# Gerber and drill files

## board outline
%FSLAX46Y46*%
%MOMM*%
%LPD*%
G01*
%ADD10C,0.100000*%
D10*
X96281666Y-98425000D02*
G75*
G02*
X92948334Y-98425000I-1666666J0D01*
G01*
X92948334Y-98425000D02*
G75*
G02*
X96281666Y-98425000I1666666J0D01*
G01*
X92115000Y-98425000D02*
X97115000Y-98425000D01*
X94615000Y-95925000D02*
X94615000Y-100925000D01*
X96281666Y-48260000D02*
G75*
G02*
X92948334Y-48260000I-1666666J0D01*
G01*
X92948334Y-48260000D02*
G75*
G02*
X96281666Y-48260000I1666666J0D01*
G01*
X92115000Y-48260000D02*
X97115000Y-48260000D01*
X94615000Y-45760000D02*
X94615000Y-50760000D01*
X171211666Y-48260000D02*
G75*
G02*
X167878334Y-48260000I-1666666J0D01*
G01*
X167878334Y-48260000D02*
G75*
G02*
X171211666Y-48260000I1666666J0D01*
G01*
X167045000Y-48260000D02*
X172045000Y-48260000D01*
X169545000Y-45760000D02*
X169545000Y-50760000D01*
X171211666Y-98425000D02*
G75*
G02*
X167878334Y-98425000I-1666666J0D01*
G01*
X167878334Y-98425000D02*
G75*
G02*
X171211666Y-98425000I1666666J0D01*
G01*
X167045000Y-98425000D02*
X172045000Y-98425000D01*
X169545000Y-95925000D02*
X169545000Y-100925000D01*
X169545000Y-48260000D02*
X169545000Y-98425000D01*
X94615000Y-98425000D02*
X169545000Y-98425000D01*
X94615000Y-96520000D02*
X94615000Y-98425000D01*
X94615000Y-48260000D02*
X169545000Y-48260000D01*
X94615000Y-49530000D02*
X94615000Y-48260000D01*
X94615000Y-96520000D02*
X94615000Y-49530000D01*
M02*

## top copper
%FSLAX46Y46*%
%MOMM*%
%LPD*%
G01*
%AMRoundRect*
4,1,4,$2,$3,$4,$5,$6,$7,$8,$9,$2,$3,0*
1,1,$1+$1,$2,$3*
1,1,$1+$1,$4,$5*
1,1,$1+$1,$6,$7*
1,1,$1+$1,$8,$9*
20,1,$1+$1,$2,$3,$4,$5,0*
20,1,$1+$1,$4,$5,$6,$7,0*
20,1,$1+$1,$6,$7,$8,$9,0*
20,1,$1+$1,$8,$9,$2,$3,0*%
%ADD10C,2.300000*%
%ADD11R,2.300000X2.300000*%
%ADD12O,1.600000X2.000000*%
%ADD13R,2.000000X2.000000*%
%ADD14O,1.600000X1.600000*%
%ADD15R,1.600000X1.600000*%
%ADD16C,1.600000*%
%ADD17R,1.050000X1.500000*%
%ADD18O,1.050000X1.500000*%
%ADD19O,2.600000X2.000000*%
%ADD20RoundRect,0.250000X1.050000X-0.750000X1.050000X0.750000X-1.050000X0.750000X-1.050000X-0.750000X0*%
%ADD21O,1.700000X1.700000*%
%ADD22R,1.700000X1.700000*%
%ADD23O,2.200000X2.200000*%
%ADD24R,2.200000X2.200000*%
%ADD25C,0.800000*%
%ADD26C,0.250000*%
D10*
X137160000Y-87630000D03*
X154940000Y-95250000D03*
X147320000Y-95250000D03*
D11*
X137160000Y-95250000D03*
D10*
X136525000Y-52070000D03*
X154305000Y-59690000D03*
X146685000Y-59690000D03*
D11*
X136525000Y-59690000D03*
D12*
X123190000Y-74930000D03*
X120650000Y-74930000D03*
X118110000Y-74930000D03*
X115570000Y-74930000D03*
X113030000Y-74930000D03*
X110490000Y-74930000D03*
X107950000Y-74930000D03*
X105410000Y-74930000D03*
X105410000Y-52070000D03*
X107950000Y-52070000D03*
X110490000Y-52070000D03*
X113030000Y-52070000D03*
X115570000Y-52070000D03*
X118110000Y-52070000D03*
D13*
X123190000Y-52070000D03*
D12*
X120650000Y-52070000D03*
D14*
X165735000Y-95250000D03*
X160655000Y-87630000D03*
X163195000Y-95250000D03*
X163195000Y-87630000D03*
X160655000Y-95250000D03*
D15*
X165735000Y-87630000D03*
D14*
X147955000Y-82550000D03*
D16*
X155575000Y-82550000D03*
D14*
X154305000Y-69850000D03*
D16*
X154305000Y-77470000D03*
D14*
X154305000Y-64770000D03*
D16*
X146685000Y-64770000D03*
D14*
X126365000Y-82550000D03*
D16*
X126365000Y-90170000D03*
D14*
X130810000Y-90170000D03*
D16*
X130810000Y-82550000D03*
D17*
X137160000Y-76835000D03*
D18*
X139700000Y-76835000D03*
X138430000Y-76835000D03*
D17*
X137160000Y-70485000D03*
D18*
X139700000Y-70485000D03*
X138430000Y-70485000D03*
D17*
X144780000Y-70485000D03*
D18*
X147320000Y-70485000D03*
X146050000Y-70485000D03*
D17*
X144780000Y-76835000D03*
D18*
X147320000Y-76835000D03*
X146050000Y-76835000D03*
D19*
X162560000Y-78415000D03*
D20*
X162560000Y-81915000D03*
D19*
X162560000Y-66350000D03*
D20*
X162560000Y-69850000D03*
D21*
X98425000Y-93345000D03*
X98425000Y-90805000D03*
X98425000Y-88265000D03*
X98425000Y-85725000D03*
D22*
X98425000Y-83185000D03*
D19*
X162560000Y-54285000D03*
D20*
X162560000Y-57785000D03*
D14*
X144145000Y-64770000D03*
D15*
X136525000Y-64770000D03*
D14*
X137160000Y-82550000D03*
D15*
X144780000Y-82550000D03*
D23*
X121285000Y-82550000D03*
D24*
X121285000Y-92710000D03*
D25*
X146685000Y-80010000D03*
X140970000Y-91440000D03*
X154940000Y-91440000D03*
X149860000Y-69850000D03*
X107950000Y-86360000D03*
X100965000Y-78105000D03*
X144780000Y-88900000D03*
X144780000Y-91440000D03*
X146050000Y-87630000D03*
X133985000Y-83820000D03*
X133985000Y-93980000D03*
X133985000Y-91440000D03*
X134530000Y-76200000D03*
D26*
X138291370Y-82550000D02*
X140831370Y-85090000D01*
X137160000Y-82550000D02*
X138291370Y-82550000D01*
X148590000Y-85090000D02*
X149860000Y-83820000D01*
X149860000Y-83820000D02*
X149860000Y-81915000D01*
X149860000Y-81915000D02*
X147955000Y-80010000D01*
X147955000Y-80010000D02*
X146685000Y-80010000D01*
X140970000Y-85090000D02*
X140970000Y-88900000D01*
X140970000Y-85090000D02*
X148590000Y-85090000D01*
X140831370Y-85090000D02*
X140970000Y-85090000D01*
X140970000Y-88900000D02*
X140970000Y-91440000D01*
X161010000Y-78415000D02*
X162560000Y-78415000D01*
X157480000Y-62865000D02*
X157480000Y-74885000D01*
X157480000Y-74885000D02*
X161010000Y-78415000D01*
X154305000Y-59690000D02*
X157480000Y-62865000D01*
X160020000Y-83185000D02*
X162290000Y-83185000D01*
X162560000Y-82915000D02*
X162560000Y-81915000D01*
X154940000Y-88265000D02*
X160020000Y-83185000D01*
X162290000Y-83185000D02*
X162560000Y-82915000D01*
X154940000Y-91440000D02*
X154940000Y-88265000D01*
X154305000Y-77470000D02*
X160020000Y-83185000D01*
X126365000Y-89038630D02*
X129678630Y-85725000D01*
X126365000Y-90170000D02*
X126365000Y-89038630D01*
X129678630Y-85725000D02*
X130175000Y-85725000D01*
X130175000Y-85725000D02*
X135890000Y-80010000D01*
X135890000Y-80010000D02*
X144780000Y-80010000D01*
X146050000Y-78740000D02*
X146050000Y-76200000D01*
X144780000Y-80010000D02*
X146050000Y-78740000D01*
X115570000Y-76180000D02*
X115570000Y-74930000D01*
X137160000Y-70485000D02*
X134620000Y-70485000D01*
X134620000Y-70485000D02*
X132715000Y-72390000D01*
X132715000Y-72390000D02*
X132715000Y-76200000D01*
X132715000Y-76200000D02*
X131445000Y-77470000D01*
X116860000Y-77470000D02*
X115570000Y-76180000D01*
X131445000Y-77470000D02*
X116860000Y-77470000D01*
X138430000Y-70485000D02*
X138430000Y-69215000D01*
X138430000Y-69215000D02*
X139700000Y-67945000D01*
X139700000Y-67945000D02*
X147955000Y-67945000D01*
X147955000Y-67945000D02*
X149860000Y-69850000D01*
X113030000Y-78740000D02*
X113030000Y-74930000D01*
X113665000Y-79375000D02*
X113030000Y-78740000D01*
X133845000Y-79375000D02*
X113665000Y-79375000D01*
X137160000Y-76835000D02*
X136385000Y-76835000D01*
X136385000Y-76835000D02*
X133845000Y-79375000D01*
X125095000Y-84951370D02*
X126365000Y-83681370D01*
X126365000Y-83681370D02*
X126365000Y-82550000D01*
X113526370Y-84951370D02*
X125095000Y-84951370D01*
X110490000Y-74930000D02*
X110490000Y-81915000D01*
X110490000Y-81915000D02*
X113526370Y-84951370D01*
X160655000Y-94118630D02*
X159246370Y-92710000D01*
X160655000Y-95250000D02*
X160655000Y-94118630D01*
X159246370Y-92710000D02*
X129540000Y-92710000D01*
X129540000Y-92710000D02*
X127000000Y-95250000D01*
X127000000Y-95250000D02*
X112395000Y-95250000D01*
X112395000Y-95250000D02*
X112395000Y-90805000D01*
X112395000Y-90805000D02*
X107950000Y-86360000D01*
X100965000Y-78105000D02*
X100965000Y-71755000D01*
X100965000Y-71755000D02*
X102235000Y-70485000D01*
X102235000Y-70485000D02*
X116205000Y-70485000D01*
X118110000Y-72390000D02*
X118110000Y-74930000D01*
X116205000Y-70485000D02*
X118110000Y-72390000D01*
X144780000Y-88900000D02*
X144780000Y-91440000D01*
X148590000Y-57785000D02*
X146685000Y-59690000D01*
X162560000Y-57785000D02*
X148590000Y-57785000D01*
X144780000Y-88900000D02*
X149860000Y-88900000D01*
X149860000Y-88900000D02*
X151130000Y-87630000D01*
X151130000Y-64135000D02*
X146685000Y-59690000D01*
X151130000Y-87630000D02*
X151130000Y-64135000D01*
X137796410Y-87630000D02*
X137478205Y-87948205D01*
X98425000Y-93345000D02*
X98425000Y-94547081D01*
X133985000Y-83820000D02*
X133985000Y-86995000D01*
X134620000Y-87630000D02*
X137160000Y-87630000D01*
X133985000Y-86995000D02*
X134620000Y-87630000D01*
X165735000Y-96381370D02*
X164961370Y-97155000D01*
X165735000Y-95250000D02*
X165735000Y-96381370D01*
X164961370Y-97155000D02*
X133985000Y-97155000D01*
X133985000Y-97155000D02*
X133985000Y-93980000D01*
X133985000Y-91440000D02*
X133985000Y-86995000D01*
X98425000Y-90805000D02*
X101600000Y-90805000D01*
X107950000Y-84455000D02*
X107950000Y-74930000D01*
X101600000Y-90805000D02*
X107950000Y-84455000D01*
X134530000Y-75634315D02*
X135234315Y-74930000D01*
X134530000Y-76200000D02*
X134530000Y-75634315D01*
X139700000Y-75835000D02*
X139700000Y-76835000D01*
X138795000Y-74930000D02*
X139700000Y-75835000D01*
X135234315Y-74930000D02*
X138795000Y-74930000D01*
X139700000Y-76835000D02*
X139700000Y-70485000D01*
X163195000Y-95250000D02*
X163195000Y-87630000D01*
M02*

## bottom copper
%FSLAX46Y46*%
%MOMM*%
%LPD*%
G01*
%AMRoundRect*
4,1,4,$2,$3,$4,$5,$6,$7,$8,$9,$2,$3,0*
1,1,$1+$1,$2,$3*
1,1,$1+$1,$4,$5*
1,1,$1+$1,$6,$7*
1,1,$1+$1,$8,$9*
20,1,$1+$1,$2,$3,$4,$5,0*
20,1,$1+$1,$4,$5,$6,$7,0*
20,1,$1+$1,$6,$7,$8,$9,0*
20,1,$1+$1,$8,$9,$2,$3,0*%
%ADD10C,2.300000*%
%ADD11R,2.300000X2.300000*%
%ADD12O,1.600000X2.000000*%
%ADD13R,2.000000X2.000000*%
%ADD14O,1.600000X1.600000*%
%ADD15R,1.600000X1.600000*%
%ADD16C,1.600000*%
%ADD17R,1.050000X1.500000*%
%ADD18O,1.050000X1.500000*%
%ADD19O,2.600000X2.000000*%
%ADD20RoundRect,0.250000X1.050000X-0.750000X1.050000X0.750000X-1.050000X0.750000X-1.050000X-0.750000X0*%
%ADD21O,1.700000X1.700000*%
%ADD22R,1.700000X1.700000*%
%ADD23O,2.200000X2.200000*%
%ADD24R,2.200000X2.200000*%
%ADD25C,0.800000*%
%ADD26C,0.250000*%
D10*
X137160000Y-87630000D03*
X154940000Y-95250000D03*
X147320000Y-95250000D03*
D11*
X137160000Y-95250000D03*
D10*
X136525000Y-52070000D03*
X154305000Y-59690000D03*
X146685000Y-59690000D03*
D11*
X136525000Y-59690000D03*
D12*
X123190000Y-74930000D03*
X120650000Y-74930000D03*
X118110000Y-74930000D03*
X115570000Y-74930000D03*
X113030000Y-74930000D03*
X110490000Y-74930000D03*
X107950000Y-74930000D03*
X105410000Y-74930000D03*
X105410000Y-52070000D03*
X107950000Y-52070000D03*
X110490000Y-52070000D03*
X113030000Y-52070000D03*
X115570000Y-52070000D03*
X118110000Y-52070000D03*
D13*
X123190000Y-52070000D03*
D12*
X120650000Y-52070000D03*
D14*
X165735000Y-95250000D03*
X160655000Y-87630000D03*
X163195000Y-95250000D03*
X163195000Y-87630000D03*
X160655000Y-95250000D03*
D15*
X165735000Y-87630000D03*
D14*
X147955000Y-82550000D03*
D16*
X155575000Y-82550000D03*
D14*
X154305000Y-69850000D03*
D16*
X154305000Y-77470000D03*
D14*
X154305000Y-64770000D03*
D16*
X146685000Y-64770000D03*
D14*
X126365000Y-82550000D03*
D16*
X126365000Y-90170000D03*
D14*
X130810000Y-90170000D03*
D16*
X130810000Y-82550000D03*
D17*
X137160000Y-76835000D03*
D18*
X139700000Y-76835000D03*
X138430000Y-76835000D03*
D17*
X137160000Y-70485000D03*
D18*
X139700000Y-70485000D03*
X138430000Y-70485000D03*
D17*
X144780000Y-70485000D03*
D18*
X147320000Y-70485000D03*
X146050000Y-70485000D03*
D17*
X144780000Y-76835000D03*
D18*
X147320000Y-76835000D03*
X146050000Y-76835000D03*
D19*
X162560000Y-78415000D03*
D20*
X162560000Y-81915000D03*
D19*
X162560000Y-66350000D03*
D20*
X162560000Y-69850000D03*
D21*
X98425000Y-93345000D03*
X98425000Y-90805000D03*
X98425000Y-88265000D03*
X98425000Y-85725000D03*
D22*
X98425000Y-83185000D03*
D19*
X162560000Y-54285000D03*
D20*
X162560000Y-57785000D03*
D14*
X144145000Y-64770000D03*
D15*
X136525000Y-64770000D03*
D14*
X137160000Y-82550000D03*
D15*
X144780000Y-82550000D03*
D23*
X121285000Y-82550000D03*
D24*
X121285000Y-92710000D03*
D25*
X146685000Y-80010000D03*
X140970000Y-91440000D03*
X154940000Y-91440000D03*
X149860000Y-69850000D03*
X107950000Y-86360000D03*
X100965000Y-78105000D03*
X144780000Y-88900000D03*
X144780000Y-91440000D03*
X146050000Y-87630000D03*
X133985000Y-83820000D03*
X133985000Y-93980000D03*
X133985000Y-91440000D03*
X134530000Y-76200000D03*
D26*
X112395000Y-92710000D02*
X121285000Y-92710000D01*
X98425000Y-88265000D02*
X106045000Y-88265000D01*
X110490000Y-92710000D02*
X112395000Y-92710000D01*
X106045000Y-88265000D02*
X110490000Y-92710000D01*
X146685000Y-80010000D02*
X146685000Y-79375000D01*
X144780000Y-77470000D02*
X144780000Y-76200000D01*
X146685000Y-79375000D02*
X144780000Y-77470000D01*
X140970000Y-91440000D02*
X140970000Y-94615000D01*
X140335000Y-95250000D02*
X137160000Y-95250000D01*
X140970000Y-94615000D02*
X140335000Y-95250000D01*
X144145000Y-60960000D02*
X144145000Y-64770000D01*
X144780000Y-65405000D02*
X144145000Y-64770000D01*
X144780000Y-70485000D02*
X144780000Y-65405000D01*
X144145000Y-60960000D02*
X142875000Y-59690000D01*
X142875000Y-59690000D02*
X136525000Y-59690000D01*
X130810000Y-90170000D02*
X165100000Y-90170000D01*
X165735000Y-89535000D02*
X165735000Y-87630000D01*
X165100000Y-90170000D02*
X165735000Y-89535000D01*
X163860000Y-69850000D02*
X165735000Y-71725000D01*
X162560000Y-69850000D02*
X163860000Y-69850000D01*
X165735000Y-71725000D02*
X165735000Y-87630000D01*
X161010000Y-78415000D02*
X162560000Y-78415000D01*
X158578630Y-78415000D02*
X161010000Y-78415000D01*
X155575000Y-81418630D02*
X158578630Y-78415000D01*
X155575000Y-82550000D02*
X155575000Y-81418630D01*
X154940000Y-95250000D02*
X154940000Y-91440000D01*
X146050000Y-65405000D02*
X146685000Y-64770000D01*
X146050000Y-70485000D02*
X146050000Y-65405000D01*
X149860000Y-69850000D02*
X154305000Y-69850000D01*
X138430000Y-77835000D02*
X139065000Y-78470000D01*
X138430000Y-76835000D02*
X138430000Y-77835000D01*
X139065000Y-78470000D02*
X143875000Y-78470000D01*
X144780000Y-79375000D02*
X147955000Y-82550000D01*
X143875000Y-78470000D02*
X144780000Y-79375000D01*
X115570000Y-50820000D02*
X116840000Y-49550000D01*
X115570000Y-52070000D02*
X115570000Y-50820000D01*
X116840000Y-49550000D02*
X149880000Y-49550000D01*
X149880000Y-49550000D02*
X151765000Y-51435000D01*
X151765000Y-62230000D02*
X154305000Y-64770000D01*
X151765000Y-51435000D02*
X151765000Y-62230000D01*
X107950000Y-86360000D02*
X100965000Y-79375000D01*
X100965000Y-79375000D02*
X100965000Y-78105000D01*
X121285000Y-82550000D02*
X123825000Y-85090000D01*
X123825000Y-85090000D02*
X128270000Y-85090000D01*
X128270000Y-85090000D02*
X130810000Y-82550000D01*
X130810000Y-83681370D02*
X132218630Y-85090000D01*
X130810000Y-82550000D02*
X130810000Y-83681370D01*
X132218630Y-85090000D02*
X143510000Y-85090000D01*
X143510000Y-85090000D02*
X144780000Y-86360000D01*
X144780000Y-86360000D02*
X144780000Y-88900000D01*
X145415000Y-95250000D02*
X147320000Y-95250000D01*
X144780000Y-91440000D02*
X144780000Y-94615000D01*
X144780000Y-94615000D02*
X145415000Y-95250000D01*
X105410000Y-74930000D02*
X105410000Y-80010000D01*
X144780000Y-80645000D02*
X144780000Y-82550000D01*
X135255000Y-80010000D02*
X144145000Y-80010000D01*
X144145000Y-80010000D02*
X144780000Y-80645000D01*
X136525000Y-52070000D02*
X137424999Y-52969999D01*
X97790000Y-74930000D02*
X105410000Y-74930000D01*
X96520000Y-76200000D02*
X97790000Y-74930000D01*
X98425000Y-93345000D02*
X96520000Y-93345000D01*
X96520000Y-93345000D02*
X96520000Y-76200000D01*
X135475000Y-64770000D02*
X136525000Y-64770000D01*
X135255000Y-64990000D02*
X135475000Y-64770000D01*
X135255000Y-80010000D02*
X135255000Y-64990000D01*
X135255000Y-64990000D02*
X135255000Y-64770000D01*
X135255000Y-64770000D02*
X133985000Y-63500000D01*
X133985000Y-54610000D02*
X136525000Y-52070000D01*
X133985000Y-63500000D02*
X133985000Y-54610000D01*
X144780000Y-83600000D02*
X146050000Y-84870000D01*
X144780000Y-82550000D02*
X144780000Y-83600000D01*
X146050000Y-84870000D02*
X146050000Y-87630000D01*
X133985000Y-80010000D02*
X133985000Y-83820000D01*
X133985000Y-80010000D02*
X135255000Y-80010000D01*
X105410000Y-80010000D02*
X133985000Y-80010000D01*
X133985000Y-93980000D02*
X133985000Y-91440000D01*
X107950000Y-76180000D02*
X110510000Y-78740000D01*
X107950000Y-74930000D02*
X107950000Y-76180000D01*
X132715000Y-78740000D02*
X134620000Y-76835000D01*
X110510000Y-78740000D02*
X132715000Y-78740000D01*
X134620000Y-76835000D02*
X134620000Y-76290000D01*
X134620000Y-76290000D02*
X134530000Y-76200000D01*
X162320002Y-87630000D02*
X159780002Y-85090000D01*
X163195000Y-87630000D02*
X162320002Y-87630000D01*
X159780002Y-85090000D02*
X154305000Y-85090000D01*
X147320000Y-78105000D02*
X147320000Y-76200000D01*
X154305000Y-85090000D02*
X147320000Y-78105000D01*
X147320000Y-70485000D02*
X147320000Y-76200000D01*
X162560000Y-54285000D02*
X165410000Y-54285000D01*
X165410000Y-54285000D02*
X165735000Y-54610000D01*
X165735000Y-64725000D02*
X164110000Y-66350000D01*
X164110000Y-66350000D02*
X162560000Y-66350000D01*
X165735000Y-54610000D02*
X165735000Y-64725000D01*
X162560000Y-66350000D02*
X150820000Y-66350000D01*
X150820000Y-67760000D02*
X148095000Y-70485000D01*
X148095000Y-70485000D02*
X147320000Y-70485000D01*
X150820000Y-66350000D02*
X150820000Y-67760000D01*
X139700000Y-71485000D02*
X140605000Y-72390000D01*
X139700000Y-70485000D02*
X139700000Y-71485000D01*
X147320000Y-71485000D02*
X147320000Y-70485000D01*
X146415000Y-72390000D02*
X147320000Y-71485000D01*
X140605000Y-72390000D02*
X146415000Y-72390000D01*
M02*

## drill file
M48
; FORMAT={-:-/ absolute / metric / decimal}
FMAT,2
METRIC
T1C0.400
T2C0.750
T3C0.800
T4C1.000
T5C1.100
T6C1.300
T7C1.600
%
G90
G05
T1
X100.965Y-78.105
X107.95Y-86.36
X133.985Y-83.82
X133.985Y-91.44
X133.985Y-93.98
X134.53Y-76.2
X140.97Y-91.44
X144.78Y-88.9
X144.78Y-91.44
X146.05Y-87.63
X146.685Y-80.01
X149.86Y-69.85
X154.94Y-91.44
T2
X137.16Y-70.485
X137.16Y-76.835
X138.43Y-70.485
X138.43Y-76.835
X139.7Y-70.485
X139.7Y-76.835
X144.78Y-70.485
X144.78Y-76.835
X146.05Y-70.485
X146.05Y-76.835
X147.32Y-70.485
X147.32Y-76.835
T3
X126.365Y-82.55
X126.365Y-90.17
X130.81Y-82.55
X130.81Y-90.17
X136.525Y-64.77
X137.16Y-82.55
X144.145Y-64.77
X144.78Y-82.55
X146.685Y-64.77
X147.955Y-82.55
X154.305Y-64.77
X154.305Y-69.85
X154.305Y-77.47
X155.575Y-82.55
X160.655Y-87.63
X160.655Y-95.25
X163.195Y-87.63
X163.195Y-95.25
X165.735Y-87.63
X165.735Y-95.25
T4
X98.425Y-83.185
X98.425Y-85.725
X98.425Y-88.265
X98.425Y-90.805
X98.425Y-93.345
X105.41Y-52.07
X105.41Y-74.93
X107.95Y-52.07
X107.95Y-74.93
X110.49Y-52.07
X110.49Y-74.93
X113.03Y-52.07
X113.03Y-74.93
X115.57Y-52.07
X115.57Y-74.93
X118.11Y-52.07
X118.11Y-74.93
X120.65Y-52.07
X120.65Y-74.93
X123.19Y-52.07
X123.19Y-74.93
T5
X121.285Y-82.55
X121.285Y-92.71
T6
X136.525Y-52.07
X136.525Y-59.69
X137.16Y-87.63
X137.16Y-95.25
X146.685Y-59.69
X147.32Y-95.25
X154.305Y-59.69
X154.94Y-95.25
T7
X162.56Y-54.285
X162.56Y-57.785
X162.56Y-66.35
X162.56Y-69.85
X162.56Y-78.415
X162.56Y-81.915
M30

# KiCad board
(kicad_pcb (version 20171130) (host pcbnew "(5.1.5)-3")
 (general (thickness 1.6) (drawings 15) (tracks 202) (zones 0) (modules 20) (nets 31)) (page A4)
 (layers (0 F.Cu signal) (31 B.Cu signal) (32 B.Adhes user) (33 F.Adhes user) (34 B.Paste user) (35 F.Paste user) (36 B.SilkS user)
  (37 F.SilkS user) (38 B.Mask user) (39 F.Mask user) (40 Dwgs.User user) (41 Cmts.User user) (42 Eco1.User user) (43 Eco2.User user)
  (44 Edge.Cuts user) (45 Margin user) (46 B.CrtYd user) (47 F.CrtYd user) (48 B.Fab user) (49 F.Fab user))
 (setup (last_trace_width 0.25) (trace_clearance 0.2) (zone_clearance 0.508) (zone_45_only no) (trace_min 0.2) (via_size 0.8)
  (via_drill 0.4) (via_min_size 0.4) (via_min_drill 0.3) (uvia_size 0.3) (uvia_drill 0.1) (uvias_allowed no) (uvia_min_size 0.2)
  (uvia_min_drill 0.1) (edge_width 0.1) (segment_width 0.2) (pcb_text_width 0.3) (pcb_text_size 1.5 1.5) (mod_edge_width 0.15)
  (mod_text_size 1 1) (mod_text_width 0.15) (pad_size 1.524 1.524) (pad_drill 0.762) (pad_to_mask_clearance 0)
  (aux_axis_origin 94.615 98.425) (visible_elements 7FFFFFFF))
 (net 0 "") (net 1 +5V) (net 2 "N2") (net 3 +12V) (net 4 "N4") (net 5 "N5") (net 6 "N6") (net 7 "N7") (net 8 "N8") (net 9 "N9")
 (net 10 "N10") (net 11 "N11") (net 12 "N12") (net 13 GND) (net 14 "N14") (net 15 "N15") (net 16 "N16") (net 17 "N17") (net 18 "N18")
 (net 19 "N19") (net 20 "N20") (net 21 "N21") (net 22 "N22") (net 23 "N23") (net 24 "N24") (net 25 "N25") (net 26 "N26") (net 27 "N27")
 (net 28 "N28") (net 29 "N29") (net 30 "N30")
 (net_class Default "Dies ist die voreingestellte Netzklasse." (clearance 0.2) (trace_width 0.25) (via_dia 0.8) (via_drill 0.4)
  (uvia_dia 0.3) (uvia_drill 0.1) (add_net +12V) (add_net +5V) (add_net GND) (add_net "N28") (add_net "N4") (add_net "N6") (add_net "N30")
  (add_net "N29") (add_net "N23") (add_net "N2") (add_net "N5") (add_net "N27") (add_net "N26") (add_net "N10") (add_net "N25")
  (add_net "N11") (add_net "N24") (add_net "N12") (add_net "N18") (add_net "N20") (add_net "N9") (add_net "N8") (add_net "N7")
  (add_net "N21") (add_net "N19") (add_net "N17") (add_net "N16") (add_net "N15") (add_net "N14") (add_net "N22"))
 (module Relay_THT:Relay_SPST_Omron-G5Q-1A (layer F.Cu) (at 137.16 95.25)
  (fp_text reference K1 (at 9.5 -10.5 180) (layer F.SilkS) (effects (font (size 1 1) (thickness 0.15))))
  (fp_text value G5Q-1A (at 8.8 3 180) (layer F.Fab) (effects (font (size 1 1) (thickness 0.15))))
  (pad 5 thru_hole circle (at 0 -7.62 180) (size 2.3 2.3) (drill 1.3) (layers *.Cu *.Mask) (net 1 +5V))
  (pad 3 thru_hole circle (at 17.78 0 180) (size 2.3 2.3) (drill 1.3) (layers *.Cu *.Mask) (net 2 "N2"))
  (pad 2 thru_hole circle (at 10.16 0 180) (size 2.3 2.3) (drill 1.3) (layers *.Cu *.Mask) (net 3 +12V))
  (pad 1 thru_hole rect (at 0 0 180) (size 2.3 2.3) (drill 1.3) (layers *.Cu *.Mask) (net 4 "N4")))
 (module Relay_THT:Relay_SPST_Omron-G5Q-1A (layer F.Cu) (at 136.525 59.69)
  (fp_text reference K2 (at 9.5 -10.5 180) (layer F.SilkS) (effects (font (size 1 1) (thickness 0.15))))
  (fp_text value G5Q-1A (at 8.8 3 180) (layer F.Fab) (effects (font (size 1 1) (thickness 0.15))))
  (pad 5 thru_hole circle (at 0 -7.62 180) (size 2.3 2.3) (drill 1.3) (layers *.Cu *.Mask) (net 1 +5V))
  (pad 3 thru_hole circle (at 17.78 0 180) (size 2.3 2.3) (drill 1.3) (layers *.Cu *.Mask) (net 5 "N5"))
  (pad 2 thru_hole circle (at 10.16 0 180) (size 2.3 2.3) (drill 1.3) (layers *.Cu *.Mask) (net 3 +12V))
  (pad 1 thru_hole rect (at 0 0 180) (size 2.3 2.3) (drill 1.3) (layers *.Cu *.Mask) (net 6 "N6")))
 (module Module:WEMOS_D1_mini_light (layer F.Cu) (at 123.19 52.07 270)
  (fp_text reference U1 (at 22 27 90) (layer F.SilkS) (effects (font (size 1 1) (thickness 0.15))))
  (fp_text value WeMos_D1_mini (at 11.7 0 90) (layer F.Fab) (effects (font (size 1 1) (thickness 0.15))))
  (pad 16 thru_hole oval (at 22.86 0 270) (size 2 1.6) (drill 1) (layers *.Cu *.Mask) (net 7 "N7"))
  (pad 15 thru_hole oval (at 22.86 2.54 270) (size 2 1.6) (drill 1) (layers *.Cu *.Mask) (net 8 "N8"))
  (pad 14 thru_hole oval (at 22.86 5.08 270) (size 2 1.6) (drill 1) (layers *.Cu *.Mask) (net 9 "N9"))
  (pad 13 thru_hole oval (at 22.86 7.62 270) (size 2 1.6) (drill 1) (layers *.Cu *.Mask) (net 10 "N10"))
  (pad 12 thru_hole oval (at 22.86 10.16 270) (size 2 1.6) (drill 1) (layers *.Cu *.Mask) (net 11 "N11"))
  (pad 11 thru_hole oval (at 22.86 12.7 270) (size 2 1.6) (drill 1) (layers *.Cu *.Mask) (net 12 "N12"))
  (pad 10 thru_hole oval (at 22.86 15.24 270) (size 2 1.6) (drill 1) (layers *.Cu *.Mask) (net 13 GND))
  (pad 9 thru_hole oval (at 22.86 17.78 270) (size 2 1.6) (drill 1) (layers *.Cu *.Mask) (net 1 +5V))
  (pad 8 thru_hole oval (at 0 17.78 270) (size 2 1.6) (drill 1) (layers *.Cu *.Mask) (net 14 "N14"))
  (pad 7 thru_hole oval (at 0 15.24 270) (size 2 1.6) (drill 1) (layers *.Cu *.Mask) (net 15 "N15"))
  (pad 6 thru_hole oval (at 0 12.7 270) (size 2 1.6) (drill 1) (layers *.Cu *.Mask) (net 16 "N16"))
  (pad 5 thru_hole oval (at 0 10.16 270) (size 2 1.6) (drill 1) (layers *.Cu *.Mask) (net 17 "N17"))
  (pad 4 thru_hole oval (at 0 7.62 270) (size 2 1.6) (drill 1) (layers *.Cu *.Mask) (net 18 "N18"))
  (pad 3 thru_hole oval (at 0 5.08 270) (size 2 1.6) (drill 1) (layers *.Cu *.Mask) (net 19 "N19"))
  (pad 1 thru_hole rect (at 0 0 270) (size 2 2) (drill 1) (layers *.Cu *.Mask) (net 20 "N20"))
  (pad 2 thru_hole oval (at 0 2.54 270) (size 2 1.6) (drill 1) (layers *.Cu *.Mask) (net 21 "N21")))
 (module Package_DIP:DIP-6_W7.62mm (layer F.Cu) (at 165.735 87.63 270)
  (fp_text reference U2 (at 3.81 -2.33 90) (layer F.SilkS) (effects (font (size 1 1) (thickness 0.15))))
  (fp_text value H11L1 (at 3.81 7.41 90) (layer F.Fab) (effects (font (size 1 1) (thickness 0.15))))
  (pad 6 thru_hole oval (at 7.62 0 270) (size 1.6 1.6) (drill 0.8) (layers *.Cu *.Mask) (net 1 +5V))
  (pad 3 thru_hole oval (at 0 5.08 270) (size 1.6 1.6) (drill 0.8) (layers *.Cu *.Mask) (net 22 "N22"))
  (pad 5 thru_hole oval (at 7.62 2.54 270) (size 1.6 1.6) (drill 0.8) (layers *.Cu *.Mask) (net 13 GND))
  (pad 2 thru_hole oval (at 0 2.54 270) (size 1.6 1.6) (drill 0.8) (layers *.Cu *.Mask) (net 13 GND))
  (pad 4 thru_hole oval (at 7.62 5.08 270) (size 1.6 1.6) (drill 0.8) (layers *.Cu *.Mask) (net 9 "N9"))
  (pad 1 thru_hole rect (at 0 0 270) (size 1.6 1.6) (drill 0.8) (layers *.Cu *.Mask) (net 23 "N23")))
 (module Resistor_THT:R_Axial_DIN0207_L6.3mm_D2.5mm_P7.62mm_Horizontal (layer F.Cu) (at 155.575 82.55 180)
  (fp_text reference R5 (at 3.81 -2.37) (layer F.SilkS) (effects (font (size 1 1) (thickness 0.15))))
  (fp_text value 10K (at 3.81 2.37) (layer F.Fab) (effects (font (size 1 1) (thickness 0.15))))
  (pad 2 thru_hole oval (at 7.62 0 180) (size 1.6 1.6) (drill 0.8) (layers *.Cu *.Mask) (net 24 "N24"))
  (pad 1 thru_hole circle (at 0 0 180) (size 1.6 1.6) (drill 0.8) (layers *.Cu *.Mask) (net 5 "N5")))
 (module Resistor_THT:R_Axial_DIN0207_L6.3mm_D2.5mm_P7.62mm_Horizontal (layer F.Cu) (at 154.305 77.47 90)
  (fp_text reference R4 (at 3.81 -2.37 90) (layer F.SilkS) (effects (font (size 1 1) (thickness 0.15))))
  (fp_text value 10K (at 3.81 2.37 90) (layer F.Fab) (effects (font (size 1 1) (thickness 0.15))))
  (pad 2 thru_hole oval (at 7.62 0 90) (size 1.6 1.6) (drill 0.8) (layers *.Cu *.Mask) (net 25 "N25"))
  (pad 1 thru_hole circle (at 0 0 90) (size 1.6 1.6) (drill 0.8) (layers *.Cu *.Mask) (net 2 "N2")))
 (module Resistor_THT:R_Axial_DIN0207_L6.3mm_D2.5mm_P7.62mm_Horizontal (layer F.Cu) (at 146.685 64.77)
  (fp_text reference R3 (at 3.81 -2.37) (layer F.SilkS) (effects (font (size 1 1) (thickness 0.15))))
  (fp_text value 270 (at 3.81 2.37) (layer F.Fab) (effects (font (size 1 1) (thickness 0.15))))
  (pad 2 thru_hole oval (at 7.62 0) (size 1.6 1.6) (drill 0.8) (layers *.Cu *.Mask) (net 18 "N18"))
  (pad 1 thru_hole circle (at 0 0) (size 1.6 1.6) (drill 0.8) (layers *.Cu *.Mask) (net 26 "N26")))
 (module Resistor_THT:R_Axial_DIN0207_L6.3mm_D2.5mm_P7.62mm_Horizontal (layer F.Cu) (at 126.365 90.17 90)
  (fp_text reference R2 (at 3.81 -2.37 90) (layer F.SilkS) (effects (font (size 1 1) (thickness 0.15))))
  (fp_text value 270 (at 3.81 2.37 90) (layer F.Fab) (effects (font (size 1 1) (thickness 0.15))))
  (pad 2 thru_hole oval (at 7.62 0 90) (size 1.6 1.6) (drill 0.8) (layers *.Cu *.Mask) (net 12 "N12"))
  (pad 1 thru_hole circle (at 0 0 90) (size 1.6 1.6) (drill 0.8) (layers *.Cu *.Mask) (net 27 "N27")))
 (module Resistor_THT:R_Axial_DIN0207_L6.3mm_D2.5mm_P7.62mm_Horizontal (layer F.Cu) (at 130.81 82.55 270)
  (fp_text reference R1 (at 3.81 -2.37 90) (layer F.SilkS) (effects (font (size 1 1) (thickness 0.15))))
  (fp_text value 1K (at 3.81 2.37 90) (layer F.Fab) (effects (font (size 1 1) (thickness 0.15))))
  (pad 2 thru_hole oval (at 7.62 0 270) (size 1.6 1.6) (drill 0.8) (layers *.Cu *.Mask) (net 23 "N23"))
  (pad 1 thru_hole circle (at 0 0 270) (size 1.6 1.6) (drill 0.8) (layers *.Cu *.Mask) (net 3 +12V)))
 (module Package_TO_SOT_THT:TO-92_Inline (layer F.Cu) (at 137.16 76.835)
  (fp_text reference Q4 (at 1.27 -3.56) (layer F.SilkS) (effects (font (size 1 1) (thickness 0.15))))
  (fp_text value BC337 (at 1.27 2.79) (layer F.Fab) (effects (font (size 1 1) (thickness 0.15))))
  (pad 1 thru_hole rect (at 0 0) (size 1.05 1.5) (drill 0.75) (layers *.Cu *.Mask) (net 11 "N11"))
  (pad 3 thru_hole oval (at 2.54 0) (size 1.05 1.5) (drill 0.75) (layers *.Cu *.Mask) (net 13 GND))
  (pad 2 thru_hole oval (at 1.27 0) (size 1.05 1.5) (drill 0.75) (layers *.Cu *.Mask) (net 24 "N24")))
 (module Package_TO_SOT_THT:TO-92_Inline (layer F.Cu) (at 137.16 70.485)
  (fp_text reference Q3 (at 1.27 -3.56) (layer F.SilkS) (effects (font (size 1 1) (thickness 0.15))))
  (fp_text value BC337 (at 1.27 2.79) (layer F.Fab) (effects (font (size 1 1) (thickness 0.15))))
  (pad 1 thru_hole rect (at 0 0) (size 1.05 1.5) (drill 0.75) (layers *.Cu *.Mask) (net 10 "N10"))
  (pad 3 thru_hole oval (at 2.54 0) (size 1.05 1.5) (drill 0.75) (layers *.Cu *.Mask) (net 13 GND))
  (pad 2 thru_hole oval (at 1.27 0) (size 1.05 1.5) (drill 0.75) (layers *.Cu *.Mask) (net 25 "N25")))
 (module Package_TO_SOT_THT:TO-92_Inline (layer F.Cu) (at 144.78 70.485)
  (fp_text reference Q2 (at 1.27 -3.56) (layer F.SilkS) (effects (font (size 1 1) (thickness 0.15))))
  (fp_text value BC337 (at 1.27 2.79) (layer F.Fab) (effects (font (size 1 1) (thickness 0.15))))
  (pad 1 thru_hole rect (at 0 0) (size 1.05 1.5) (drill 0.75) (layers *.Cu *.Mask) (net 6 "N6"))
  (pad 3 thru_hole oval (at 2.54 0) (size 1.05 1.5) (drill 0.75) (layers *.Cu *.Mask) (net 13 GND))
  (pad 2 thru_hole oval (at 1.27 0) (size 1.05 1.5) (drill 0.75) (layers *.Cu *.Mask) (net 26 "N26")))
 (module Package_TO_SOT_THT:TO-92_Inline (layer F.Cu) (at 144.78 76.835)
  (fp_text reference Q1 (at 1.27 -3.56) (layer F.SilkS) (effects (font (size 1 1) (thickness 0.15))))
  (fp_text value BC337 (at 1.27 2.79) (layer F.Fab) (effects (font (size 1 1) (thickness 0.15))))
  (pad 1 thru_hole rect (at 0 0) (size 1.05 1.5) (drill 0.75) (layers *.Cu *.Mask) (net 4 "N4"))
  (pad 3 thru_hole oval (at 2.54 0) (size 1.05 1.5) (drill 0.75) (layers *.Cu *.Mask) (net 13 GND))
  (pad 2 thru_hole oval (at 1.27 0) (size 1.05 1.5) (drill 0.75) (layers *.Cu *.Mask) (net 27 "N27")))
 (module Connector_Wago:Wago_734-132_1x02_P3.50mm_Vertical (layer F.Cu) (at 162.56 81.915 90)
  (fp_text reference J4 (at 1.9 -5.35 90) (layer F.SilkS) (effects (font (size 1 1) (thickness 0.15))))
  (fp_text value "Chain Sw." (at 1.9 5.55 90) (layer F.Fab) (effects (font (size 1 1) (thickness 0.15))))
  (pad 2 thru_hole oval (at 3.5 0 90) (size 2 2.6) (drill 1.6) (layers *.Cu *.Mask) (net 5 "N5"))
  (pad 1 thru_hole roundrect (at 0 0 90) (size 2 2.6) (drill 1.6) (layers *.Cu *.Mask) (roundrect_rratio 0.125) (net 2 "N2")))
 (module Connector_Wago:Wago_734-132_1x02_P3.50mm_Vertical (layer F.Cu) (at 162.56 69.85 90)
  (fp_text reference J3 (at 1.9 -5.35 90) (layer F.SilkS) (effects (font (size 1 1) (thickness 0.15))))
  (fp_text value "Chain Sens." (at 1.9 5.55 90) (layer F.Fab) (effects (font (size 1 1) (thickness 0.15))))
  (pad 2 thru_hole oval (at 3.5 0 90) (size 2 2.6) (drill 1.6) (layers *.Cu *.Mask) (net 13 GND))
  (pad 1 thru_hole roundrect (at 0 0 90) (size 2 2.6) (drill 1.6) (layers *.Cu *.Mask) (roundrect_rratio 0.125) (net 23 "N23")))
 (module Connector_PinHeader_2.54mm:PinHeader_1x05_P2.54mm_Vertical (layer F.Cu) (at 98.425 83.185)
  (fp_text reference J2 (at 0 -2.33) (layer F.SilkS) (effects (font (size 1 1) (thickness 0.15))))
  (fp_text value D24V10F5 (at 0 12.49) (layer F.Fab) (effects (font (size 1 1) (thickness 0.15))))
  (pad 5 thru_hole oval (at 0 10.16) (size 1.7 1.7) (drill 1) (layers *.Cu *.Mask) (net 1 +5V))
  (pad 4 thru_hole oval (at 0 7.62) (size 1.7 1.7) (drill 1) (layers *.Cu *.Mask) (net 13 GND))
  (pad 3 thru_hole oval (at 0 5.08) (size 1.7 1.7) (drill 1) (layers *.Cu *.Mask) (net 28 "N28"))
  (pad 2 thru_hole oval (at 0 2.54) (size 1.7 1.7) (drill 1) (layers *.Cu *.Mask) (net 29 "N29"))
  (pad 1 thru_hole rect (at 0 0) (size 1.7 1.7) (drill 1) (layers *.Cu *.Mask) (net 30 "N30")))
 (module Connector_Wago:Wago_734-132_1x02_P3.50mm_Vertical (layer F.Cu) (at 162.56 57.785 90)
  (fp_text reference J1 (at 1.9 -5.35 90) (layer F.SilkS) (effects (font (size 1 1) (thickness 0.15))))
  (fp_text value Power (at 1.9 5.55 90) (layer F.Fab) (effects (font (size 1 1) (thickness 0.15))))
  (pad 2 thru_hole oval (at 3.5 0 90) (size 2 2.6) (drill 1.6) (layers *.Cu *.Mask) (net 13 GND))
  (pad 1 thru_hole roundrect (at 0 0 90) (size 2 2.6) (drill 1.6) (layers *.Cu *.Mask) (roundrect_rratio 0.125) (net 3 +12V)))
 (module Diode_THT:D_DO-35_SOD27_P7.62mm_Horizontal (layer F.Cu) (at 136.525 64.77)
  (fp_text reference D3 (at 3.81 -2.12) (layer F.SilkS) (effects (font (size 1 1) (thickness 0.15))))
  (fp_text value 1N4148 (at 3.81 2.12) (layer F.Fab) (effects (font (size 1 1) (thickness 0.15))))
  (pad 2 thru_hole oval (at 7.62 0) (size 1.6 1.6) (drill 0.8) (layers *.Cu *.Mask) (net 6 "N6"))
  (pad 1 thru_hole rect (at 0 0) (size 1.6 1.6) (drill 0.8) (layers *.Cu *.Mask) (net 1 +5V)))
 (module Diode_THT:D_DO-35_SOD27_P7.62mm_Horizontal (layer F.Cu) (at 144.78 82.55 180)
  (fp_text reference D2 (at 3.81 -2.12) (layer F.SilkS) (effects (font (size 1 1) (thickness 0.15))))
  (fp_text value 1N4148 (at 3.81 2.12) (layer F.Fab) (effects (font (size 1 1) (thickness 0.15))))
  (pad 2 thru_hole oval (at 7.62 0 180) (size 1.6 1.6) (drill 0.8) (layers *.Cu *.Mask) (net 4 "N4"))
  (pad 1 thru_hole rect (at 0 0 180) (size 1.6 1.6) (drill 0.8) (layers *.Cu *.Mask) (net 1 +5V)))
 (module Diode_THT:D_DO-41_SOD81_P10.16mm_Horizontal (layer F.Cu) (at 121.285 92.71 90)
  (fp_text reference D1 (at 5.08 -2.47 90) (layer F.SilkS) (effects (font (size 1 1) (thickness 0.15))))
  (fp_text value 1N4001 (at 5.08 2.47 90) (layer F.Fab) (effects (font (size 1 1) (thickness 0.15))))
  (pad 2 thru_hole oval (at 10.16 0 90) (size 2.2 2.2) (drill 1.1) (layers *.Cu *.Mask) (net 3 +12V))
  (pad 1 thru_hole rect (at 0 0 90) (size 2.2 2.2) (drill 1.1) (layers *.Cu *.Mask) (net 28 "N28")))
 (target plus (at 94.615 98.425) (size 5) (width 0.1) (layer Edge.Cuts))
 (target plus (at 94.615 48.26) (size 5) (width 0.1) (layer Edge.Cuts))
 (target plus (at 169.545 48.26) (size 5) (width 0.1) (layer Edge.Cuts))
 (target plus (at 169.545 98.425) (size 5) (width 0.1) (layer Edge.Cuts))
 (gr_line (start 169.545 48.26) (end 169.545 98.425) (layer Edge.Cuts) (width 0.1))
 (gr_line (start 94.615 98.425) (end 169.545 98.425) (layer Edge.Cuts) (width 0.1))
 (gr_line (start 94.615 96.52) (end 94.615 98.425) (layer Edge.Cuts) (width 0.1))
 (gr_line (start 94.615 48.26) (end 169.545 48.26) (layer Edge.Cuts) (width 0.1))
 (gr_line (start 94.615 49.53) (end 94.615 48.26) (layer Edge.Cuts) (width 0.1))
 (gr_line (start 94.615 96.52) (end 94.615 49.53) (layer Edge.Cuts) (width 0.1))
 (segment (start 112.395 92.71) (end 121.285 92.71) (width 0.25) (layer B.Cu) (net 28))
 (segment (start 98.425 88.265) (end 106.045 88.265) (width 0.25) (layer B.Cu) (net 28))
 (segment (start 110.49 92.71) (end 112.395 92.71) (width 0.25) (layer B.Cu) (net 28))
 (segment (start 106.045 88.265) (end 110.49 92.71) (width 0.25) (layer B.Cu) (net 28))
 (segment (start 138.29137 82.55) (end 140.83137 85.09) (width 0.25) (layer F.Cu) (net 4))
 (segment (start 137.16 82.55) (end 138.29137 82.55) (width 0.25) (layer F.Cu) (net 4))
 (segment (start 148.59 85.09) (end 149.86 83.82) (width 0.25) (layer F.Cu) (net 4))
 (segment (start 149.86 83.82) (end 149.86 81.915) (width 0.25) (layer F.Cu) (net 4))
 (segment (start 149.86 81.915) (end 147.955 80.01) (width 0.25) (layer F.Cu) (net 4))
 (via (at 146.685 80.01) (size 0.8) (drill 0.4) (layers F.Cu B.Cu) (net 4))
 (segment (start 147.955 80.01) (end 146.685 80.01) (width 0.25) (layer F.Cu) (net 4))
 (segment (start 146.685 80.01) (end 146.685 79.375) (width 0.25) (layer B.Cu) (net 4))
 (segment (start 144.78 77.47) (end 144.78 76.2) (width 0.25) (layer B.Cu) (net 4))
 (segment (start 146.685 79.375) (end 144.78 77.47) (width 0.25) (layer B.Cu) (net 4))
 (segment (start 140.97 85.09) (end 140.97 88.9) (width 0.25) (layer F.Cu) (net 4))
 (segment (start 140.97 85.09) (end 148.59 85.09) (width 0.25) (layer F.Cu) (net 4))
 (segment (start 140.83137 85.09) (end 140.97 85.09) (width 0.25) (layer F.Cu) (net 4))
 (segment (start 140.97 88.9) (end 140.97 91.44) (width 0.25) (layer F.Cu) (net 4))
 (via (at 140.97 91.44) (size 0.8) (drill 0.4) (layers F.Cu B.Cu) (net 4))
 (segment (start 140.97 91.44) (end 140.97 94.615) (width 0.25) (layer B.Cu) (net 4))
 (segment (start 140.335 95.25) (end 137.16 95.25) (width 0.25) (layer B.Cu) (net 4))
 (segment (start 140.97 94.615) (end 140.335 95.25) (width 0.25) (layer B.Cu) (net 4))
 (segment (start 144.145 60.96) (end 144.145 64.77) (width 0.25) (layer B.Cu) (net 6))
 (segment (start 144.78 65.405) (end 144.145 64.77) (width 0.25) (layer B.Cu) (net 6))
 (segment (start 144.78 70.485) (end 144.78 65.405) (width 0.25) (layer B.Cu) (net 6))
 (segment (start 144.145 60.96) (end 142.875 59.69) (width 0.25) (layer B.Cu) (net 6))
 (segment (start 142.875 59.69) (end 136.525 59.69) (width 0.25) (layer B.Cu) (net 6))
 (segment (start 130.81 90.17) (end 165.1 90.17) (width 0.25) (layer B.Cu) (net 23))
 (segment (start 165.735 89.535) (end 165.735 87.63) (width 0.25) (layer B.Cu) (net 23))
 (segment (start 165.1 90.17) (end 165.735 89.535) (width 0.25) (layer B.Cu) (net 23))
 (segment (start 163.86 69.85) (end 165.735 71.725) (width 0.25) (layer B.Cu) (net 23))
 (segment (start 162.56 69.85) (end 163.86 69.85) (width 0.25) (layer B.Cu) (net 23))
 (segment (start 165.735 71.725) (end 165.735 87.63) (width 0.25) (layer B.Cu) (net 23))
 (segment (start 161.01 78.415) (end 162.56 78.415) (width 0.25) (layer B.Cu) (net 5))
 (segment (start 158.57863 78.415) (end 161.01 78.415) (width 0.25) (layer B.Cu) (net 5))
 (segment (start 155.575 81.41863) (end 158.57863 78.415) (width 0.25) (layer B.Cu) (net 5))
 (segment (start 155.575 82.55) (end 155.575 81.41863) (width 0.25) (layer B.Cu) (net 5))
 (segment (start 161.01 78.415) (end 162.56 78.415) (width 0.25) (layer F.Cu) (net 5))
 (segment (start 157.48 62.865) (end 157.48 74.885) (width 0.25) (layer F.Cu) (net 5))
 (segment (start 157.48 74.885) (end 161.01 78.415) (width 0.25) (layer F.Cu) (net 5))
 (segment (start 154.305 59.69) (end 157.48 62.865) (width 0.25) (layer F.Cu) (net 5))
 (segment (start 154.94 95.25) (end 154.94 91.44) (width 0.25) (layer B.Cu) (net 2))
 (via (at 154.94 91.44) (size 0.8) (drill 0.4) (layers F.Cu B.Cu) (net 2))
 (segment (start 160.02 83.185) (end 162.29 83.185) (width 0.25) (layer F.Cu) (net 2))
 (segment (start 162.56 82.915) (end 162.56 81.915) (width 0.25) (layer F.Cu) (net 2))
 (segment (start 154.94 88.265) (end 160.02 83.185) (width 0.25) (layer F.Cu) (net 2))
 (segment (start 162.29 83.185) (end 162.56 82.915) (width 0.25) (layer F.Cu) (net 2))
 (segment (start 154.94 91.44) (end 154.94 88.265) (width 0.25) (layer F.Cu) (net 2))
 (segment (start 154.305 77.47) (end 160.02 83.185) (width 0.25) (layer F.Cu) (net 2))
 (segment (start 126.365 89.03863) (end 129.67863 85.725) (width 0.25) (layer F.Cu) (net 27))
 (segment (start 126.365 90.17) (end 126.365 89.03863) (width 0.25) (layer F.Cu) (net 27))
 (segment (start 129.67863 85.725) (end 130.175 85.725) (width 0.25) (layer F.Cu) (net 27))
 (segment (start 130.175 85.725) (end 135.89 80.01) (width 0.25) (layer F.Cu) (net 27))
 (segment (start 135.89 80.01) (end 144.78 80.01) (width 0.25) (layer F.Cu) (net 27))
 (segment (start 146.05 78.74) (end 146.05 76.2) (width 0.25) (layer F.Cu) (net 27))
 (segment (start 144.78 80.01) (end 146.05 78.74) (width 0.25) (layer F.Cu) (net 27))
 (segment (start 146.05 65.405) (end 146.685 64.77) (width 0.25) (layer B.Cu) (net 26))
 (segment (start 146.05 70.485) (end 146.05 65.405) (width 0.25) (layer B.Cu) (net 26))
 (segment (start 115.57 76.18) (end 115.57 74.93) (width 0.25) (layer F.Cu) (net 10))
 (segment (start 137.16 70.485) (end 134.62 70.485) (width 0.25) (layer F.Cu) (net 10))
 (segment (start 134.62 70.485) (end 132.715 72.39) (width 0.25) (layer F.Cu) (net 10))
 (segment (start 132.715 72.39) (end 132.715 76.2) (width 0.25) (layer F.Cu) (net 10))
 (segment (start 132.715 76.2) (end 131.445 77.47) (width 0.25) (layer F.Cu) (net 10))
 (segment (start 116.86 77.47) (end 115.57 76.18) (width 0.25) (layer F.Cu) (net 10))
 (segment (start 131.445 77.47) (end 116.86 77.47) (width 0.25) (layer F.Cu) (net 10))
 (segment (start 138.43 70.485) (end 138.43 69.215) (width 0.25) (layer F.Cu) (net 25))
 (segment (start 138.43 69.215) (end 139.7 67.945) (width 0.25) (layer F.Cu) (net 25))
 (segment (start 139.7 67.945) (end 147.955 67.945) (width 0.25) (layer F.Cu) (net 25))
 (via (at 149.86 69.85) (size 0.8) (drill 0.4) (layers F.Cu B.Cu) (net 25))
 (segment (start 147.955 67.945) (end 149.86 69.85) (width 0.25) (layer F.Cu) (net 25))
 (segment (start 149.86 69.85) (end 154.305 69.85) (width 0.25) (layer B.Cu) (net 25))
 (segment (start 113.03 78.74) (end 113.03 74.93) (width 0.25) (layer F.Cu) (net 11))
 (segment (start 113.665 79.375) (end 113.03 78.74) (width 0.25) (layer F.Cu) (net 11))
 (segment (start 133.845 79.375) (end 113.665 79.375) (width 0.25) (layer F.Cu) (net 11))
 (segment (start 137.16 76.835) (end 136.385 76.835) (width 0.25) (layer F.Cu) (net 11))
 (segment (start 136.385 76.835) (end 133.845 79.375) (width 0.25) (layer F.Cu) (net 11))
 (segment (start 138.43 77.835) (end 139.065 78.47) (width 0.25) (layer B.Cu) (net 24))
 (segment (start 138.43 76.835) (end 138.43 77.835) (width 0.25) (layer B.Cu) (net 24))
 (segment (start 139.065 78.47) (end 143.875 78.47) (width 0.25) (layer B.Cu) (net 24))
 (segment (start 144.78 79.375) (end 147.955 82.55) (width 0.25) (layer B.Cu) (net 24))
 (segment (start 143.875 78.47) (end 144.78 79.375) (width 0.25) (layer B.Cu) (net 24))
 (segment (start 125.095 84.95137) (end 126.365 83.68137) (width 0.25) (layer F.Cu) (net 12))
 (segment (start 126.365 83.68137) (end 126.365 82.55) (width 0.25) (layer F.Cu) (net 12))
 (segment (start 113.52637 84.95137) (end 125.095 84.95137) (width 0.25) (layer F.Cu) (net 12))
 (segment (start 110.49 74.93) (end 110.49 81.915) (width 0.25) (layer F.Cu) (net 12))
 (segment (start 110.49 81.915) (end 113.52637 84.95137) (width 0.25) (layer F.Cu) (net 12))
 (segment (start 115.57 50.82) (end 116.84 49.55) (width 0.25) (layer B.Cu) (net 18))
 (segment (start 115.57 52.07) (end 115.57 50.82) (width 0.25) (layer B.Cu) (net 18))
 (segment (start 116.84 49.55) (end 149.88 49.55) (width 0.25) (layer B.Cu) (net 18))
 (segment (start 149.88 49.55) (end 151.765 51.435) (width 0.25) (layer B.Cu) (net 18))
 (segment (start 151.765 62.23) (end 154.305 64.77) (width 0.25) (layer B.Cu) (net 18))
 (segment (start 151.765 51.435) (end 151.765 62.23) (width 0.25) (layer B.Cu) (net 18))
 (segment (start 160.655 94.11863) (end 159.24637 92.71) (width 0.25) (layer F.Cu) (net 9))
 (segment (start 160.655 95.25) (end 160.655 94.11863) (width 0.25) (layer F.Cu) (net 9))
 (segment (start 159.24637 92.71) (end 129.54 92.71) (width 0.25) (layer F.Cu) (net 9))
 (segment (start 129.54 92.71) (end 127 95.25) (width 0.25) (layer F.Cu) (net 9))
 (segment (start 127 95.25) (end 112.395 95.25) (width 0.25) (layer F.Cu) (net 9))
 (segment (start 112.395 95.25) (end 112.395 90.805) (width 0.25) (layer F.Cu) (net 9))
 (via (at 107.95 86.36) (size 0.8) (drill 0.4) (layers F.Cu B.Cu) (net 9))
 (segment (start 112.395 90.805) (end 107.95 86.36) (width 0.25) (layer F.Cu) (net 9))
 (segment (start 107.95 86.36) (end 100.965 79.375) (width 0.25) (layer B.Cu) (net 9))
 (via (at 100.965 78.105) (size 0.8) (drill 0.4) (layers F.Cu B.Cu) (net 9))
 (segment (start 100.965 79.375) (end 100.965 78.105) (width 0.25) (layer B.Cu) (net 9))
 (segment (start 100.965 78.105) (end 100.965 71.755) (width 0.25) (layer F.Cu) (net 9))
 (segment (start 100.965 71.755) (end 102.235 70.485) (width 0.25) (layer F.Cu) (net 9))
 (segment (start 102.235 70.485) (end 116.205 70.485) (width 0.25) (layer F.Cu) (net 9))
 (segment (start 118.11 72.39) (end 118.11 74.93) (width 0.25) (layer F.Cu) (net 9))
 (segment (start 116.205 70.485) (end 118.11 72.39) (width 0.25) (layer F.Cu) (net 9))
 (segment (start 121.285 82.55) (end 123.825 85.09) (width 0.25) (layer B.Cu) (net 3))
 (segment (start 123.825 85.09) (end 128.27 85.09) (width 0.25) (layer B.Cu) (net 3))
 (segment (start 128.27 85.09) (end 130.81 82.55) (width 0.25) (layer B.Cu) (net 3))
 (segment (start 130.81 83.68137) (end 132.21863 85.09) (width 0.25) (layer B.Cu) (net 3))
 (segment (start 130.81 82.55) (end 130.81 83.68137) (width 0.25) (layer B.Cu) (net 3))
 (segment (start 132.21863 85.09) (end 143.51 85.09) (width 0.25) (layer B.Cu) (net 3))
 (segment (start 143.51 85.09) (end 144.78 86.36) (width 0.25) (layer B.Cu) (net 3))
 (via (at 144.78 88.9) (size 0.8) (drill 0.4) (layers F.Cu B.Cu) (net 3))
 (segment (start 144.78 86.36) (end 144.78 88.9) (width 0.25) (layer B.Cu) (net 3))
 (segment (start 144.78 88.9) (end 144.78 91.44) (width 0.25) (layer F.Cu) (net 3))
 (via (at 144.78 91.44) (size 0.8) (drill 0.4) (layers F.Cu B.Cu) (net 3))
 (segment (start 145.415 95.25) (end 147.32 95.25) (width 0.25) (layer B.Cu) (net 3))
 (segment (start 144.78 91.44) (end 144.78 94.615) (width 0.25) (layer B.Cu) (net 3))
 (segment (start 144.78 94.615) (end 145.415 95.25) (width 0.25) (layer B.Cu) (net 3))
 (segment (start 148.59 57.785) (end 146.685 59.69) (width 0.25) (layer F.Cu) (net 3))
 (segment (start 162.56 57.785) (end 148.59 57.785) (width 0.25) (layer F.Cu) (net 3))
 (segment (start 144.78 88.9) (end 149.86 88.9) (width 0.25) (layer F.Cu) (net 3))
 (segment (start 149.86 88.9) (end 151.13 87.63) (width 0.25) (layer F.Cu) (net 3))
 (segment (start 151.13 64.135) (end 146.685 59.69) (width 0.25) (layer F.Cu) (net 3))
 (segment (start 151.13 87.63) (end 151.13 64.135) (width 0.25) (layer F.Cu) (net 3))
 (segment (start 105.41 74.93) (end 105.41 80.01) (width 0.25) (layer B.Cu) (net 1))
 (segment (start 144.78 80.645) (end 144.78 82.55) (width 0.25) (layer B.Cu) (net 1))
 (segment (start 135.255 80.01) (end 144.145 80.01) (width 0.25) (layer B.Cu) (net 1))
 (segment (start 144.145 80.01) (end 144.78 80.645) (width 0.25) (layer B.Cu) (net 1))
 (segment (start 136.525 52.07) (end 137.424999 52.969999) (width 0.25) (layer B.Cu) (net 1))
 (segment (start 97.79 74.93) (end 105.41 74.93) (width 0.25) (layer B.Cu) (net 1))
 (segment (start 96.52 76.2) (end 97.79 74.93) (width 0.25) (layer B.Cu) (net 1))
 (segment (start 98.425 93.345) (end 96.52 93.345) (width 0.25) (layer B.Cu) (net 1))
 (segment (start 96.52 93.345) (end 96.52 76.2) (width 0.25) (layer B.Cu) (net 1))
 (segment (start 135.475 64.77) (end 136.525 64.77) (width 0.25) (layer B.Cu) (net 1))
 (segment (start 135.255 64.99) (end 135.475 64.77) (width 0.25) (layer B.Cu) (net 1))
 (segment (start 135.255 80.01) (end 135.255 64.99) (width 0.25) (layer B.Cu) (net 1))
 (segment (start 135.255 64.99) (end 135.255 64.77) (width 0.25) (layer B.Cu) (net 1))
 (segment (start 135.255 64.77) (end 133.985 63.5) (width 0.25) (layer B.Cu) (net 1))
 (segment (start 133.985 54.61) (end 136.525 52.07) (width 0.25) (layer B.Cu) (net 1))
 (segment (start 133.985 63.5) (end 133.985 54.61) (width 0.25) (layer B.Cu) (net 1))
 (segment (start 144.78 83.6) (end 146.05 84.87) (width 0.25) (layer B.Cu) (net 1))
 (segment (start 144.78 82.55) (end 144.78 83.6) (width 0.25) (layer B.Cu) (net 1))
 (via (at 146.05 87.63) (size 0.8) (drill 0.4) (layers F.Cu B.Cu) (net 1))
 (segment (start 146.05 84.87) (end 146.05 87.63) (width 0.25) (layer B.Cu) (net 1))
 (segment (start 137.79641 87.63) (end 137.478205 87.948205) (width 0.25) (layer F.Cu) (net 1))
 (segment (start 98.425 93.345) (end 98.425 94.547081) (width 0.25) (layer F.Cu) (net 1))
 (segment (start 133.985 80.01) (end 133.985 83.82) (width 0.25) (layer B.Cu) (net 1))
 (segment (start 133.985 80.01) (end 135.255 80.01) (width 0.25) (layer B.Cu) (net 1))
 (segment (start 105.41 80.01) (end 133.985 80.01) (width 0.25) (layer B.Cu) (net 1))
 (via (at 133.985 83.82) (size 0.8) (drill 0.4) (layers F.Cu B.Cu) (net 1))
 (segment (start 133.985 83.82) (end 133.985 86.995) (width 0.25) (layer F.Cu) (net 1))
 (segment (start 134.62 87.63) (end 137.16 87.63) (width 0.25) (layer F.Cu) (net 1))
 (segment (start 133.985 86.995) (end 134.62 87.63) (width 0.25) (layer F.Cu) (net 1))
 (segment (start 165.735 96.38137) (end 164.96137 97.155) (width 0.25) (layer F.Cu) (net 1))
 (segment (start 165.735 95.25) (end 165.735 96.38137) (width 0.25) (layer F.Cu) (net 1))
 (segment (start 164.96137 97.155) (end 133.985 97.155) (width 0.25) (layer F.Cu) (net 1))
 (segment (start 133.985 97.155) (end 133.985 93.98) (width 0.25) (layer F.Cu) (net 1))
 (via (at 133.985 93.98) (size 0.8) (drill 0.4) (layers F.Cu B.Cu) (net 1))
 (segment (start 133.985 93.98) (end 133.985 91.44) (width 0.25) (layer B.Cu) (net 1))
 (via (at 133.985 91.44) (size 0.8) (drill 0.4) (layers F.Cu B.Cu) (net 1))
 (segment (start 133.985 91.44) (end 133.985 86.995) (width 0.25) (layer F.Cu) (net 1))
 (segment (start 98.425 90.805) (end 101.6 90.805) (width 0.25) (layer F.Cu) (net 13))
 (segment (start 107.95 84.455) (end 107.95 74.93) (width 0.25) (layer F.Cu) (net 13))
 (segment (start 101.6 90.805) (end 107.95 84.455) (width 0.25) (layer F.Cu) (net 13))
 (segment (start 107.95 76.18) (end 110.51 78.74) (width 0.25) (layer B.Cu) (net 13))
 (segment (start 107.95 74.93) (end 107.95 76.18) (width 0.25) (layer B.Cu) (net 13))
 (segment (start 132.715 78.74) (end 134.62 76.835) (width 0.25) (layer B.Cu) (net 13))
 (segment (start 110.51 78.74) (end 132.715 78.74) (width 0.25) (layer B.Cu) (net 13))
 (segment (start 134.62 76.835) (end 134.62 76.29) (width 0.25) (layer B.Cu) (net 13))
 (via (at 134.53 76.2) (size 0.8) (drill 0.4) (layers F.Cu B.Cu) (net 13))
 (segment (start 134.62 76.29) (end 134.53 76.2) (width 0.25) (layer B.Cu) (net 13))
 (segment (start 134.53 75.634315) (end 135.234315 74.93) (width 0.25) (layer F.Cu) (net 13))
 (segment (start 134.53 76.2) (end 134.53 75.634315) (width 0.25) (layer F.Cu) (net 13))
 (segment (start 139.7 75.835) (end 139.7 76.835) (width 0.25) (layer F.Cu) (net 13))
 (segment (start 138.795 74.93) (end 139.7 75.835) (width 0.25) (layer F.Cu) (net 13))
 (segment (start 135.234315 74.93) (end 138.795 74.93) (width 0.25) (layer F.Cu) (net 13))
 (segment (start 139.7 76.835) (end 139.7 70.485) (width 0.25) (layer F.Cu) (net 13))
 (segment (start 163.195 95.25) (end 163.195 87.63) (width 0.25) (layer F.Cu) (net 13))
 (segment (start 162.320002 87.63) (end 159.780002 85.09) (width 0.25) (layer B.Cu) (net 13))
 (segment (start 163.195 87.63) (end 162.320002 87.63) (width 0.25) (layer B.Cu) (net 13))
 (segment (start 159.780002 85.09) (end 154.305 85.09) (width 0.25) (layer B.Cu) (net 13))
 (segment (start 147.32 78.105) (end 147.32 76.2) (width 0.25) (layer B.Cu) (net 13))
 (segment (start 154.305 85.09) (end 147.32 78.105) (width 0.25) (layer B.Cu) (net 13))
 (segment (start 147.32 70.485) (end 147.32 76.2) (width 0.25) (layer B.Cu) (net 13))
 (segment (start 162.56 54.285) (end 165.41 54.285) (width 0.25) (layer B.Cu) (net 13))
 (segment (start 165.41 54.285) (end 165.735 54.61) (width 0.25) (layer B.Cu) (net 13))
 (segment (start 165.735 64.725) (end 164.11 66.35) (width 0.25) (layer B.Cu) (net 13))
 (segment (start 164.11 66.35) (end 162.56 66.35) (width 0.25) (layer B.Cu) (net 13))
 (segment (start 165.735 54.61) (end 165.735 64.725) (width 0.25) (layer B.Cu) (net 13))
 (segment (start 162.56 66.35) (end 150.82 66.35) (width 0.25) (layer B.Cu) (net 13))
 (segment (start 150.82 67.76) (end 148.095 70.485) (width 0.25) (layer B.Cu) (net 13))
 (segment (start 148.095 70.485) (end 147.32 70.485) (width 0.25) (layer B.Cu) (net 13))
 (segment (start 150.82 66.35) (end 150.82 67.76) (width 0.25) (layer B.Cu) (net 13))
 (segment (start 139.7 71.485) (end 140.605 72.39) (width 0.25) (layer B.Cu) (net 13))
 (segment (start 139.7 70.485) (end 139.7 71.485) (width 0.25) (layer B.Cu) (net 13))
 (segment (start 147.32 71.485) (end 147.32 70.485) (width 0.25) (layer B.Cu) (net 13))
 (segment (start 146.415 72.39) (end 147.32 71.485) (width 0.25) (layer B.Cu) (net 13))
 (segment (start 140.605 72.39) (end 146.415 72.39) (width 0.25) (layer B.Cu) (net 13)))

